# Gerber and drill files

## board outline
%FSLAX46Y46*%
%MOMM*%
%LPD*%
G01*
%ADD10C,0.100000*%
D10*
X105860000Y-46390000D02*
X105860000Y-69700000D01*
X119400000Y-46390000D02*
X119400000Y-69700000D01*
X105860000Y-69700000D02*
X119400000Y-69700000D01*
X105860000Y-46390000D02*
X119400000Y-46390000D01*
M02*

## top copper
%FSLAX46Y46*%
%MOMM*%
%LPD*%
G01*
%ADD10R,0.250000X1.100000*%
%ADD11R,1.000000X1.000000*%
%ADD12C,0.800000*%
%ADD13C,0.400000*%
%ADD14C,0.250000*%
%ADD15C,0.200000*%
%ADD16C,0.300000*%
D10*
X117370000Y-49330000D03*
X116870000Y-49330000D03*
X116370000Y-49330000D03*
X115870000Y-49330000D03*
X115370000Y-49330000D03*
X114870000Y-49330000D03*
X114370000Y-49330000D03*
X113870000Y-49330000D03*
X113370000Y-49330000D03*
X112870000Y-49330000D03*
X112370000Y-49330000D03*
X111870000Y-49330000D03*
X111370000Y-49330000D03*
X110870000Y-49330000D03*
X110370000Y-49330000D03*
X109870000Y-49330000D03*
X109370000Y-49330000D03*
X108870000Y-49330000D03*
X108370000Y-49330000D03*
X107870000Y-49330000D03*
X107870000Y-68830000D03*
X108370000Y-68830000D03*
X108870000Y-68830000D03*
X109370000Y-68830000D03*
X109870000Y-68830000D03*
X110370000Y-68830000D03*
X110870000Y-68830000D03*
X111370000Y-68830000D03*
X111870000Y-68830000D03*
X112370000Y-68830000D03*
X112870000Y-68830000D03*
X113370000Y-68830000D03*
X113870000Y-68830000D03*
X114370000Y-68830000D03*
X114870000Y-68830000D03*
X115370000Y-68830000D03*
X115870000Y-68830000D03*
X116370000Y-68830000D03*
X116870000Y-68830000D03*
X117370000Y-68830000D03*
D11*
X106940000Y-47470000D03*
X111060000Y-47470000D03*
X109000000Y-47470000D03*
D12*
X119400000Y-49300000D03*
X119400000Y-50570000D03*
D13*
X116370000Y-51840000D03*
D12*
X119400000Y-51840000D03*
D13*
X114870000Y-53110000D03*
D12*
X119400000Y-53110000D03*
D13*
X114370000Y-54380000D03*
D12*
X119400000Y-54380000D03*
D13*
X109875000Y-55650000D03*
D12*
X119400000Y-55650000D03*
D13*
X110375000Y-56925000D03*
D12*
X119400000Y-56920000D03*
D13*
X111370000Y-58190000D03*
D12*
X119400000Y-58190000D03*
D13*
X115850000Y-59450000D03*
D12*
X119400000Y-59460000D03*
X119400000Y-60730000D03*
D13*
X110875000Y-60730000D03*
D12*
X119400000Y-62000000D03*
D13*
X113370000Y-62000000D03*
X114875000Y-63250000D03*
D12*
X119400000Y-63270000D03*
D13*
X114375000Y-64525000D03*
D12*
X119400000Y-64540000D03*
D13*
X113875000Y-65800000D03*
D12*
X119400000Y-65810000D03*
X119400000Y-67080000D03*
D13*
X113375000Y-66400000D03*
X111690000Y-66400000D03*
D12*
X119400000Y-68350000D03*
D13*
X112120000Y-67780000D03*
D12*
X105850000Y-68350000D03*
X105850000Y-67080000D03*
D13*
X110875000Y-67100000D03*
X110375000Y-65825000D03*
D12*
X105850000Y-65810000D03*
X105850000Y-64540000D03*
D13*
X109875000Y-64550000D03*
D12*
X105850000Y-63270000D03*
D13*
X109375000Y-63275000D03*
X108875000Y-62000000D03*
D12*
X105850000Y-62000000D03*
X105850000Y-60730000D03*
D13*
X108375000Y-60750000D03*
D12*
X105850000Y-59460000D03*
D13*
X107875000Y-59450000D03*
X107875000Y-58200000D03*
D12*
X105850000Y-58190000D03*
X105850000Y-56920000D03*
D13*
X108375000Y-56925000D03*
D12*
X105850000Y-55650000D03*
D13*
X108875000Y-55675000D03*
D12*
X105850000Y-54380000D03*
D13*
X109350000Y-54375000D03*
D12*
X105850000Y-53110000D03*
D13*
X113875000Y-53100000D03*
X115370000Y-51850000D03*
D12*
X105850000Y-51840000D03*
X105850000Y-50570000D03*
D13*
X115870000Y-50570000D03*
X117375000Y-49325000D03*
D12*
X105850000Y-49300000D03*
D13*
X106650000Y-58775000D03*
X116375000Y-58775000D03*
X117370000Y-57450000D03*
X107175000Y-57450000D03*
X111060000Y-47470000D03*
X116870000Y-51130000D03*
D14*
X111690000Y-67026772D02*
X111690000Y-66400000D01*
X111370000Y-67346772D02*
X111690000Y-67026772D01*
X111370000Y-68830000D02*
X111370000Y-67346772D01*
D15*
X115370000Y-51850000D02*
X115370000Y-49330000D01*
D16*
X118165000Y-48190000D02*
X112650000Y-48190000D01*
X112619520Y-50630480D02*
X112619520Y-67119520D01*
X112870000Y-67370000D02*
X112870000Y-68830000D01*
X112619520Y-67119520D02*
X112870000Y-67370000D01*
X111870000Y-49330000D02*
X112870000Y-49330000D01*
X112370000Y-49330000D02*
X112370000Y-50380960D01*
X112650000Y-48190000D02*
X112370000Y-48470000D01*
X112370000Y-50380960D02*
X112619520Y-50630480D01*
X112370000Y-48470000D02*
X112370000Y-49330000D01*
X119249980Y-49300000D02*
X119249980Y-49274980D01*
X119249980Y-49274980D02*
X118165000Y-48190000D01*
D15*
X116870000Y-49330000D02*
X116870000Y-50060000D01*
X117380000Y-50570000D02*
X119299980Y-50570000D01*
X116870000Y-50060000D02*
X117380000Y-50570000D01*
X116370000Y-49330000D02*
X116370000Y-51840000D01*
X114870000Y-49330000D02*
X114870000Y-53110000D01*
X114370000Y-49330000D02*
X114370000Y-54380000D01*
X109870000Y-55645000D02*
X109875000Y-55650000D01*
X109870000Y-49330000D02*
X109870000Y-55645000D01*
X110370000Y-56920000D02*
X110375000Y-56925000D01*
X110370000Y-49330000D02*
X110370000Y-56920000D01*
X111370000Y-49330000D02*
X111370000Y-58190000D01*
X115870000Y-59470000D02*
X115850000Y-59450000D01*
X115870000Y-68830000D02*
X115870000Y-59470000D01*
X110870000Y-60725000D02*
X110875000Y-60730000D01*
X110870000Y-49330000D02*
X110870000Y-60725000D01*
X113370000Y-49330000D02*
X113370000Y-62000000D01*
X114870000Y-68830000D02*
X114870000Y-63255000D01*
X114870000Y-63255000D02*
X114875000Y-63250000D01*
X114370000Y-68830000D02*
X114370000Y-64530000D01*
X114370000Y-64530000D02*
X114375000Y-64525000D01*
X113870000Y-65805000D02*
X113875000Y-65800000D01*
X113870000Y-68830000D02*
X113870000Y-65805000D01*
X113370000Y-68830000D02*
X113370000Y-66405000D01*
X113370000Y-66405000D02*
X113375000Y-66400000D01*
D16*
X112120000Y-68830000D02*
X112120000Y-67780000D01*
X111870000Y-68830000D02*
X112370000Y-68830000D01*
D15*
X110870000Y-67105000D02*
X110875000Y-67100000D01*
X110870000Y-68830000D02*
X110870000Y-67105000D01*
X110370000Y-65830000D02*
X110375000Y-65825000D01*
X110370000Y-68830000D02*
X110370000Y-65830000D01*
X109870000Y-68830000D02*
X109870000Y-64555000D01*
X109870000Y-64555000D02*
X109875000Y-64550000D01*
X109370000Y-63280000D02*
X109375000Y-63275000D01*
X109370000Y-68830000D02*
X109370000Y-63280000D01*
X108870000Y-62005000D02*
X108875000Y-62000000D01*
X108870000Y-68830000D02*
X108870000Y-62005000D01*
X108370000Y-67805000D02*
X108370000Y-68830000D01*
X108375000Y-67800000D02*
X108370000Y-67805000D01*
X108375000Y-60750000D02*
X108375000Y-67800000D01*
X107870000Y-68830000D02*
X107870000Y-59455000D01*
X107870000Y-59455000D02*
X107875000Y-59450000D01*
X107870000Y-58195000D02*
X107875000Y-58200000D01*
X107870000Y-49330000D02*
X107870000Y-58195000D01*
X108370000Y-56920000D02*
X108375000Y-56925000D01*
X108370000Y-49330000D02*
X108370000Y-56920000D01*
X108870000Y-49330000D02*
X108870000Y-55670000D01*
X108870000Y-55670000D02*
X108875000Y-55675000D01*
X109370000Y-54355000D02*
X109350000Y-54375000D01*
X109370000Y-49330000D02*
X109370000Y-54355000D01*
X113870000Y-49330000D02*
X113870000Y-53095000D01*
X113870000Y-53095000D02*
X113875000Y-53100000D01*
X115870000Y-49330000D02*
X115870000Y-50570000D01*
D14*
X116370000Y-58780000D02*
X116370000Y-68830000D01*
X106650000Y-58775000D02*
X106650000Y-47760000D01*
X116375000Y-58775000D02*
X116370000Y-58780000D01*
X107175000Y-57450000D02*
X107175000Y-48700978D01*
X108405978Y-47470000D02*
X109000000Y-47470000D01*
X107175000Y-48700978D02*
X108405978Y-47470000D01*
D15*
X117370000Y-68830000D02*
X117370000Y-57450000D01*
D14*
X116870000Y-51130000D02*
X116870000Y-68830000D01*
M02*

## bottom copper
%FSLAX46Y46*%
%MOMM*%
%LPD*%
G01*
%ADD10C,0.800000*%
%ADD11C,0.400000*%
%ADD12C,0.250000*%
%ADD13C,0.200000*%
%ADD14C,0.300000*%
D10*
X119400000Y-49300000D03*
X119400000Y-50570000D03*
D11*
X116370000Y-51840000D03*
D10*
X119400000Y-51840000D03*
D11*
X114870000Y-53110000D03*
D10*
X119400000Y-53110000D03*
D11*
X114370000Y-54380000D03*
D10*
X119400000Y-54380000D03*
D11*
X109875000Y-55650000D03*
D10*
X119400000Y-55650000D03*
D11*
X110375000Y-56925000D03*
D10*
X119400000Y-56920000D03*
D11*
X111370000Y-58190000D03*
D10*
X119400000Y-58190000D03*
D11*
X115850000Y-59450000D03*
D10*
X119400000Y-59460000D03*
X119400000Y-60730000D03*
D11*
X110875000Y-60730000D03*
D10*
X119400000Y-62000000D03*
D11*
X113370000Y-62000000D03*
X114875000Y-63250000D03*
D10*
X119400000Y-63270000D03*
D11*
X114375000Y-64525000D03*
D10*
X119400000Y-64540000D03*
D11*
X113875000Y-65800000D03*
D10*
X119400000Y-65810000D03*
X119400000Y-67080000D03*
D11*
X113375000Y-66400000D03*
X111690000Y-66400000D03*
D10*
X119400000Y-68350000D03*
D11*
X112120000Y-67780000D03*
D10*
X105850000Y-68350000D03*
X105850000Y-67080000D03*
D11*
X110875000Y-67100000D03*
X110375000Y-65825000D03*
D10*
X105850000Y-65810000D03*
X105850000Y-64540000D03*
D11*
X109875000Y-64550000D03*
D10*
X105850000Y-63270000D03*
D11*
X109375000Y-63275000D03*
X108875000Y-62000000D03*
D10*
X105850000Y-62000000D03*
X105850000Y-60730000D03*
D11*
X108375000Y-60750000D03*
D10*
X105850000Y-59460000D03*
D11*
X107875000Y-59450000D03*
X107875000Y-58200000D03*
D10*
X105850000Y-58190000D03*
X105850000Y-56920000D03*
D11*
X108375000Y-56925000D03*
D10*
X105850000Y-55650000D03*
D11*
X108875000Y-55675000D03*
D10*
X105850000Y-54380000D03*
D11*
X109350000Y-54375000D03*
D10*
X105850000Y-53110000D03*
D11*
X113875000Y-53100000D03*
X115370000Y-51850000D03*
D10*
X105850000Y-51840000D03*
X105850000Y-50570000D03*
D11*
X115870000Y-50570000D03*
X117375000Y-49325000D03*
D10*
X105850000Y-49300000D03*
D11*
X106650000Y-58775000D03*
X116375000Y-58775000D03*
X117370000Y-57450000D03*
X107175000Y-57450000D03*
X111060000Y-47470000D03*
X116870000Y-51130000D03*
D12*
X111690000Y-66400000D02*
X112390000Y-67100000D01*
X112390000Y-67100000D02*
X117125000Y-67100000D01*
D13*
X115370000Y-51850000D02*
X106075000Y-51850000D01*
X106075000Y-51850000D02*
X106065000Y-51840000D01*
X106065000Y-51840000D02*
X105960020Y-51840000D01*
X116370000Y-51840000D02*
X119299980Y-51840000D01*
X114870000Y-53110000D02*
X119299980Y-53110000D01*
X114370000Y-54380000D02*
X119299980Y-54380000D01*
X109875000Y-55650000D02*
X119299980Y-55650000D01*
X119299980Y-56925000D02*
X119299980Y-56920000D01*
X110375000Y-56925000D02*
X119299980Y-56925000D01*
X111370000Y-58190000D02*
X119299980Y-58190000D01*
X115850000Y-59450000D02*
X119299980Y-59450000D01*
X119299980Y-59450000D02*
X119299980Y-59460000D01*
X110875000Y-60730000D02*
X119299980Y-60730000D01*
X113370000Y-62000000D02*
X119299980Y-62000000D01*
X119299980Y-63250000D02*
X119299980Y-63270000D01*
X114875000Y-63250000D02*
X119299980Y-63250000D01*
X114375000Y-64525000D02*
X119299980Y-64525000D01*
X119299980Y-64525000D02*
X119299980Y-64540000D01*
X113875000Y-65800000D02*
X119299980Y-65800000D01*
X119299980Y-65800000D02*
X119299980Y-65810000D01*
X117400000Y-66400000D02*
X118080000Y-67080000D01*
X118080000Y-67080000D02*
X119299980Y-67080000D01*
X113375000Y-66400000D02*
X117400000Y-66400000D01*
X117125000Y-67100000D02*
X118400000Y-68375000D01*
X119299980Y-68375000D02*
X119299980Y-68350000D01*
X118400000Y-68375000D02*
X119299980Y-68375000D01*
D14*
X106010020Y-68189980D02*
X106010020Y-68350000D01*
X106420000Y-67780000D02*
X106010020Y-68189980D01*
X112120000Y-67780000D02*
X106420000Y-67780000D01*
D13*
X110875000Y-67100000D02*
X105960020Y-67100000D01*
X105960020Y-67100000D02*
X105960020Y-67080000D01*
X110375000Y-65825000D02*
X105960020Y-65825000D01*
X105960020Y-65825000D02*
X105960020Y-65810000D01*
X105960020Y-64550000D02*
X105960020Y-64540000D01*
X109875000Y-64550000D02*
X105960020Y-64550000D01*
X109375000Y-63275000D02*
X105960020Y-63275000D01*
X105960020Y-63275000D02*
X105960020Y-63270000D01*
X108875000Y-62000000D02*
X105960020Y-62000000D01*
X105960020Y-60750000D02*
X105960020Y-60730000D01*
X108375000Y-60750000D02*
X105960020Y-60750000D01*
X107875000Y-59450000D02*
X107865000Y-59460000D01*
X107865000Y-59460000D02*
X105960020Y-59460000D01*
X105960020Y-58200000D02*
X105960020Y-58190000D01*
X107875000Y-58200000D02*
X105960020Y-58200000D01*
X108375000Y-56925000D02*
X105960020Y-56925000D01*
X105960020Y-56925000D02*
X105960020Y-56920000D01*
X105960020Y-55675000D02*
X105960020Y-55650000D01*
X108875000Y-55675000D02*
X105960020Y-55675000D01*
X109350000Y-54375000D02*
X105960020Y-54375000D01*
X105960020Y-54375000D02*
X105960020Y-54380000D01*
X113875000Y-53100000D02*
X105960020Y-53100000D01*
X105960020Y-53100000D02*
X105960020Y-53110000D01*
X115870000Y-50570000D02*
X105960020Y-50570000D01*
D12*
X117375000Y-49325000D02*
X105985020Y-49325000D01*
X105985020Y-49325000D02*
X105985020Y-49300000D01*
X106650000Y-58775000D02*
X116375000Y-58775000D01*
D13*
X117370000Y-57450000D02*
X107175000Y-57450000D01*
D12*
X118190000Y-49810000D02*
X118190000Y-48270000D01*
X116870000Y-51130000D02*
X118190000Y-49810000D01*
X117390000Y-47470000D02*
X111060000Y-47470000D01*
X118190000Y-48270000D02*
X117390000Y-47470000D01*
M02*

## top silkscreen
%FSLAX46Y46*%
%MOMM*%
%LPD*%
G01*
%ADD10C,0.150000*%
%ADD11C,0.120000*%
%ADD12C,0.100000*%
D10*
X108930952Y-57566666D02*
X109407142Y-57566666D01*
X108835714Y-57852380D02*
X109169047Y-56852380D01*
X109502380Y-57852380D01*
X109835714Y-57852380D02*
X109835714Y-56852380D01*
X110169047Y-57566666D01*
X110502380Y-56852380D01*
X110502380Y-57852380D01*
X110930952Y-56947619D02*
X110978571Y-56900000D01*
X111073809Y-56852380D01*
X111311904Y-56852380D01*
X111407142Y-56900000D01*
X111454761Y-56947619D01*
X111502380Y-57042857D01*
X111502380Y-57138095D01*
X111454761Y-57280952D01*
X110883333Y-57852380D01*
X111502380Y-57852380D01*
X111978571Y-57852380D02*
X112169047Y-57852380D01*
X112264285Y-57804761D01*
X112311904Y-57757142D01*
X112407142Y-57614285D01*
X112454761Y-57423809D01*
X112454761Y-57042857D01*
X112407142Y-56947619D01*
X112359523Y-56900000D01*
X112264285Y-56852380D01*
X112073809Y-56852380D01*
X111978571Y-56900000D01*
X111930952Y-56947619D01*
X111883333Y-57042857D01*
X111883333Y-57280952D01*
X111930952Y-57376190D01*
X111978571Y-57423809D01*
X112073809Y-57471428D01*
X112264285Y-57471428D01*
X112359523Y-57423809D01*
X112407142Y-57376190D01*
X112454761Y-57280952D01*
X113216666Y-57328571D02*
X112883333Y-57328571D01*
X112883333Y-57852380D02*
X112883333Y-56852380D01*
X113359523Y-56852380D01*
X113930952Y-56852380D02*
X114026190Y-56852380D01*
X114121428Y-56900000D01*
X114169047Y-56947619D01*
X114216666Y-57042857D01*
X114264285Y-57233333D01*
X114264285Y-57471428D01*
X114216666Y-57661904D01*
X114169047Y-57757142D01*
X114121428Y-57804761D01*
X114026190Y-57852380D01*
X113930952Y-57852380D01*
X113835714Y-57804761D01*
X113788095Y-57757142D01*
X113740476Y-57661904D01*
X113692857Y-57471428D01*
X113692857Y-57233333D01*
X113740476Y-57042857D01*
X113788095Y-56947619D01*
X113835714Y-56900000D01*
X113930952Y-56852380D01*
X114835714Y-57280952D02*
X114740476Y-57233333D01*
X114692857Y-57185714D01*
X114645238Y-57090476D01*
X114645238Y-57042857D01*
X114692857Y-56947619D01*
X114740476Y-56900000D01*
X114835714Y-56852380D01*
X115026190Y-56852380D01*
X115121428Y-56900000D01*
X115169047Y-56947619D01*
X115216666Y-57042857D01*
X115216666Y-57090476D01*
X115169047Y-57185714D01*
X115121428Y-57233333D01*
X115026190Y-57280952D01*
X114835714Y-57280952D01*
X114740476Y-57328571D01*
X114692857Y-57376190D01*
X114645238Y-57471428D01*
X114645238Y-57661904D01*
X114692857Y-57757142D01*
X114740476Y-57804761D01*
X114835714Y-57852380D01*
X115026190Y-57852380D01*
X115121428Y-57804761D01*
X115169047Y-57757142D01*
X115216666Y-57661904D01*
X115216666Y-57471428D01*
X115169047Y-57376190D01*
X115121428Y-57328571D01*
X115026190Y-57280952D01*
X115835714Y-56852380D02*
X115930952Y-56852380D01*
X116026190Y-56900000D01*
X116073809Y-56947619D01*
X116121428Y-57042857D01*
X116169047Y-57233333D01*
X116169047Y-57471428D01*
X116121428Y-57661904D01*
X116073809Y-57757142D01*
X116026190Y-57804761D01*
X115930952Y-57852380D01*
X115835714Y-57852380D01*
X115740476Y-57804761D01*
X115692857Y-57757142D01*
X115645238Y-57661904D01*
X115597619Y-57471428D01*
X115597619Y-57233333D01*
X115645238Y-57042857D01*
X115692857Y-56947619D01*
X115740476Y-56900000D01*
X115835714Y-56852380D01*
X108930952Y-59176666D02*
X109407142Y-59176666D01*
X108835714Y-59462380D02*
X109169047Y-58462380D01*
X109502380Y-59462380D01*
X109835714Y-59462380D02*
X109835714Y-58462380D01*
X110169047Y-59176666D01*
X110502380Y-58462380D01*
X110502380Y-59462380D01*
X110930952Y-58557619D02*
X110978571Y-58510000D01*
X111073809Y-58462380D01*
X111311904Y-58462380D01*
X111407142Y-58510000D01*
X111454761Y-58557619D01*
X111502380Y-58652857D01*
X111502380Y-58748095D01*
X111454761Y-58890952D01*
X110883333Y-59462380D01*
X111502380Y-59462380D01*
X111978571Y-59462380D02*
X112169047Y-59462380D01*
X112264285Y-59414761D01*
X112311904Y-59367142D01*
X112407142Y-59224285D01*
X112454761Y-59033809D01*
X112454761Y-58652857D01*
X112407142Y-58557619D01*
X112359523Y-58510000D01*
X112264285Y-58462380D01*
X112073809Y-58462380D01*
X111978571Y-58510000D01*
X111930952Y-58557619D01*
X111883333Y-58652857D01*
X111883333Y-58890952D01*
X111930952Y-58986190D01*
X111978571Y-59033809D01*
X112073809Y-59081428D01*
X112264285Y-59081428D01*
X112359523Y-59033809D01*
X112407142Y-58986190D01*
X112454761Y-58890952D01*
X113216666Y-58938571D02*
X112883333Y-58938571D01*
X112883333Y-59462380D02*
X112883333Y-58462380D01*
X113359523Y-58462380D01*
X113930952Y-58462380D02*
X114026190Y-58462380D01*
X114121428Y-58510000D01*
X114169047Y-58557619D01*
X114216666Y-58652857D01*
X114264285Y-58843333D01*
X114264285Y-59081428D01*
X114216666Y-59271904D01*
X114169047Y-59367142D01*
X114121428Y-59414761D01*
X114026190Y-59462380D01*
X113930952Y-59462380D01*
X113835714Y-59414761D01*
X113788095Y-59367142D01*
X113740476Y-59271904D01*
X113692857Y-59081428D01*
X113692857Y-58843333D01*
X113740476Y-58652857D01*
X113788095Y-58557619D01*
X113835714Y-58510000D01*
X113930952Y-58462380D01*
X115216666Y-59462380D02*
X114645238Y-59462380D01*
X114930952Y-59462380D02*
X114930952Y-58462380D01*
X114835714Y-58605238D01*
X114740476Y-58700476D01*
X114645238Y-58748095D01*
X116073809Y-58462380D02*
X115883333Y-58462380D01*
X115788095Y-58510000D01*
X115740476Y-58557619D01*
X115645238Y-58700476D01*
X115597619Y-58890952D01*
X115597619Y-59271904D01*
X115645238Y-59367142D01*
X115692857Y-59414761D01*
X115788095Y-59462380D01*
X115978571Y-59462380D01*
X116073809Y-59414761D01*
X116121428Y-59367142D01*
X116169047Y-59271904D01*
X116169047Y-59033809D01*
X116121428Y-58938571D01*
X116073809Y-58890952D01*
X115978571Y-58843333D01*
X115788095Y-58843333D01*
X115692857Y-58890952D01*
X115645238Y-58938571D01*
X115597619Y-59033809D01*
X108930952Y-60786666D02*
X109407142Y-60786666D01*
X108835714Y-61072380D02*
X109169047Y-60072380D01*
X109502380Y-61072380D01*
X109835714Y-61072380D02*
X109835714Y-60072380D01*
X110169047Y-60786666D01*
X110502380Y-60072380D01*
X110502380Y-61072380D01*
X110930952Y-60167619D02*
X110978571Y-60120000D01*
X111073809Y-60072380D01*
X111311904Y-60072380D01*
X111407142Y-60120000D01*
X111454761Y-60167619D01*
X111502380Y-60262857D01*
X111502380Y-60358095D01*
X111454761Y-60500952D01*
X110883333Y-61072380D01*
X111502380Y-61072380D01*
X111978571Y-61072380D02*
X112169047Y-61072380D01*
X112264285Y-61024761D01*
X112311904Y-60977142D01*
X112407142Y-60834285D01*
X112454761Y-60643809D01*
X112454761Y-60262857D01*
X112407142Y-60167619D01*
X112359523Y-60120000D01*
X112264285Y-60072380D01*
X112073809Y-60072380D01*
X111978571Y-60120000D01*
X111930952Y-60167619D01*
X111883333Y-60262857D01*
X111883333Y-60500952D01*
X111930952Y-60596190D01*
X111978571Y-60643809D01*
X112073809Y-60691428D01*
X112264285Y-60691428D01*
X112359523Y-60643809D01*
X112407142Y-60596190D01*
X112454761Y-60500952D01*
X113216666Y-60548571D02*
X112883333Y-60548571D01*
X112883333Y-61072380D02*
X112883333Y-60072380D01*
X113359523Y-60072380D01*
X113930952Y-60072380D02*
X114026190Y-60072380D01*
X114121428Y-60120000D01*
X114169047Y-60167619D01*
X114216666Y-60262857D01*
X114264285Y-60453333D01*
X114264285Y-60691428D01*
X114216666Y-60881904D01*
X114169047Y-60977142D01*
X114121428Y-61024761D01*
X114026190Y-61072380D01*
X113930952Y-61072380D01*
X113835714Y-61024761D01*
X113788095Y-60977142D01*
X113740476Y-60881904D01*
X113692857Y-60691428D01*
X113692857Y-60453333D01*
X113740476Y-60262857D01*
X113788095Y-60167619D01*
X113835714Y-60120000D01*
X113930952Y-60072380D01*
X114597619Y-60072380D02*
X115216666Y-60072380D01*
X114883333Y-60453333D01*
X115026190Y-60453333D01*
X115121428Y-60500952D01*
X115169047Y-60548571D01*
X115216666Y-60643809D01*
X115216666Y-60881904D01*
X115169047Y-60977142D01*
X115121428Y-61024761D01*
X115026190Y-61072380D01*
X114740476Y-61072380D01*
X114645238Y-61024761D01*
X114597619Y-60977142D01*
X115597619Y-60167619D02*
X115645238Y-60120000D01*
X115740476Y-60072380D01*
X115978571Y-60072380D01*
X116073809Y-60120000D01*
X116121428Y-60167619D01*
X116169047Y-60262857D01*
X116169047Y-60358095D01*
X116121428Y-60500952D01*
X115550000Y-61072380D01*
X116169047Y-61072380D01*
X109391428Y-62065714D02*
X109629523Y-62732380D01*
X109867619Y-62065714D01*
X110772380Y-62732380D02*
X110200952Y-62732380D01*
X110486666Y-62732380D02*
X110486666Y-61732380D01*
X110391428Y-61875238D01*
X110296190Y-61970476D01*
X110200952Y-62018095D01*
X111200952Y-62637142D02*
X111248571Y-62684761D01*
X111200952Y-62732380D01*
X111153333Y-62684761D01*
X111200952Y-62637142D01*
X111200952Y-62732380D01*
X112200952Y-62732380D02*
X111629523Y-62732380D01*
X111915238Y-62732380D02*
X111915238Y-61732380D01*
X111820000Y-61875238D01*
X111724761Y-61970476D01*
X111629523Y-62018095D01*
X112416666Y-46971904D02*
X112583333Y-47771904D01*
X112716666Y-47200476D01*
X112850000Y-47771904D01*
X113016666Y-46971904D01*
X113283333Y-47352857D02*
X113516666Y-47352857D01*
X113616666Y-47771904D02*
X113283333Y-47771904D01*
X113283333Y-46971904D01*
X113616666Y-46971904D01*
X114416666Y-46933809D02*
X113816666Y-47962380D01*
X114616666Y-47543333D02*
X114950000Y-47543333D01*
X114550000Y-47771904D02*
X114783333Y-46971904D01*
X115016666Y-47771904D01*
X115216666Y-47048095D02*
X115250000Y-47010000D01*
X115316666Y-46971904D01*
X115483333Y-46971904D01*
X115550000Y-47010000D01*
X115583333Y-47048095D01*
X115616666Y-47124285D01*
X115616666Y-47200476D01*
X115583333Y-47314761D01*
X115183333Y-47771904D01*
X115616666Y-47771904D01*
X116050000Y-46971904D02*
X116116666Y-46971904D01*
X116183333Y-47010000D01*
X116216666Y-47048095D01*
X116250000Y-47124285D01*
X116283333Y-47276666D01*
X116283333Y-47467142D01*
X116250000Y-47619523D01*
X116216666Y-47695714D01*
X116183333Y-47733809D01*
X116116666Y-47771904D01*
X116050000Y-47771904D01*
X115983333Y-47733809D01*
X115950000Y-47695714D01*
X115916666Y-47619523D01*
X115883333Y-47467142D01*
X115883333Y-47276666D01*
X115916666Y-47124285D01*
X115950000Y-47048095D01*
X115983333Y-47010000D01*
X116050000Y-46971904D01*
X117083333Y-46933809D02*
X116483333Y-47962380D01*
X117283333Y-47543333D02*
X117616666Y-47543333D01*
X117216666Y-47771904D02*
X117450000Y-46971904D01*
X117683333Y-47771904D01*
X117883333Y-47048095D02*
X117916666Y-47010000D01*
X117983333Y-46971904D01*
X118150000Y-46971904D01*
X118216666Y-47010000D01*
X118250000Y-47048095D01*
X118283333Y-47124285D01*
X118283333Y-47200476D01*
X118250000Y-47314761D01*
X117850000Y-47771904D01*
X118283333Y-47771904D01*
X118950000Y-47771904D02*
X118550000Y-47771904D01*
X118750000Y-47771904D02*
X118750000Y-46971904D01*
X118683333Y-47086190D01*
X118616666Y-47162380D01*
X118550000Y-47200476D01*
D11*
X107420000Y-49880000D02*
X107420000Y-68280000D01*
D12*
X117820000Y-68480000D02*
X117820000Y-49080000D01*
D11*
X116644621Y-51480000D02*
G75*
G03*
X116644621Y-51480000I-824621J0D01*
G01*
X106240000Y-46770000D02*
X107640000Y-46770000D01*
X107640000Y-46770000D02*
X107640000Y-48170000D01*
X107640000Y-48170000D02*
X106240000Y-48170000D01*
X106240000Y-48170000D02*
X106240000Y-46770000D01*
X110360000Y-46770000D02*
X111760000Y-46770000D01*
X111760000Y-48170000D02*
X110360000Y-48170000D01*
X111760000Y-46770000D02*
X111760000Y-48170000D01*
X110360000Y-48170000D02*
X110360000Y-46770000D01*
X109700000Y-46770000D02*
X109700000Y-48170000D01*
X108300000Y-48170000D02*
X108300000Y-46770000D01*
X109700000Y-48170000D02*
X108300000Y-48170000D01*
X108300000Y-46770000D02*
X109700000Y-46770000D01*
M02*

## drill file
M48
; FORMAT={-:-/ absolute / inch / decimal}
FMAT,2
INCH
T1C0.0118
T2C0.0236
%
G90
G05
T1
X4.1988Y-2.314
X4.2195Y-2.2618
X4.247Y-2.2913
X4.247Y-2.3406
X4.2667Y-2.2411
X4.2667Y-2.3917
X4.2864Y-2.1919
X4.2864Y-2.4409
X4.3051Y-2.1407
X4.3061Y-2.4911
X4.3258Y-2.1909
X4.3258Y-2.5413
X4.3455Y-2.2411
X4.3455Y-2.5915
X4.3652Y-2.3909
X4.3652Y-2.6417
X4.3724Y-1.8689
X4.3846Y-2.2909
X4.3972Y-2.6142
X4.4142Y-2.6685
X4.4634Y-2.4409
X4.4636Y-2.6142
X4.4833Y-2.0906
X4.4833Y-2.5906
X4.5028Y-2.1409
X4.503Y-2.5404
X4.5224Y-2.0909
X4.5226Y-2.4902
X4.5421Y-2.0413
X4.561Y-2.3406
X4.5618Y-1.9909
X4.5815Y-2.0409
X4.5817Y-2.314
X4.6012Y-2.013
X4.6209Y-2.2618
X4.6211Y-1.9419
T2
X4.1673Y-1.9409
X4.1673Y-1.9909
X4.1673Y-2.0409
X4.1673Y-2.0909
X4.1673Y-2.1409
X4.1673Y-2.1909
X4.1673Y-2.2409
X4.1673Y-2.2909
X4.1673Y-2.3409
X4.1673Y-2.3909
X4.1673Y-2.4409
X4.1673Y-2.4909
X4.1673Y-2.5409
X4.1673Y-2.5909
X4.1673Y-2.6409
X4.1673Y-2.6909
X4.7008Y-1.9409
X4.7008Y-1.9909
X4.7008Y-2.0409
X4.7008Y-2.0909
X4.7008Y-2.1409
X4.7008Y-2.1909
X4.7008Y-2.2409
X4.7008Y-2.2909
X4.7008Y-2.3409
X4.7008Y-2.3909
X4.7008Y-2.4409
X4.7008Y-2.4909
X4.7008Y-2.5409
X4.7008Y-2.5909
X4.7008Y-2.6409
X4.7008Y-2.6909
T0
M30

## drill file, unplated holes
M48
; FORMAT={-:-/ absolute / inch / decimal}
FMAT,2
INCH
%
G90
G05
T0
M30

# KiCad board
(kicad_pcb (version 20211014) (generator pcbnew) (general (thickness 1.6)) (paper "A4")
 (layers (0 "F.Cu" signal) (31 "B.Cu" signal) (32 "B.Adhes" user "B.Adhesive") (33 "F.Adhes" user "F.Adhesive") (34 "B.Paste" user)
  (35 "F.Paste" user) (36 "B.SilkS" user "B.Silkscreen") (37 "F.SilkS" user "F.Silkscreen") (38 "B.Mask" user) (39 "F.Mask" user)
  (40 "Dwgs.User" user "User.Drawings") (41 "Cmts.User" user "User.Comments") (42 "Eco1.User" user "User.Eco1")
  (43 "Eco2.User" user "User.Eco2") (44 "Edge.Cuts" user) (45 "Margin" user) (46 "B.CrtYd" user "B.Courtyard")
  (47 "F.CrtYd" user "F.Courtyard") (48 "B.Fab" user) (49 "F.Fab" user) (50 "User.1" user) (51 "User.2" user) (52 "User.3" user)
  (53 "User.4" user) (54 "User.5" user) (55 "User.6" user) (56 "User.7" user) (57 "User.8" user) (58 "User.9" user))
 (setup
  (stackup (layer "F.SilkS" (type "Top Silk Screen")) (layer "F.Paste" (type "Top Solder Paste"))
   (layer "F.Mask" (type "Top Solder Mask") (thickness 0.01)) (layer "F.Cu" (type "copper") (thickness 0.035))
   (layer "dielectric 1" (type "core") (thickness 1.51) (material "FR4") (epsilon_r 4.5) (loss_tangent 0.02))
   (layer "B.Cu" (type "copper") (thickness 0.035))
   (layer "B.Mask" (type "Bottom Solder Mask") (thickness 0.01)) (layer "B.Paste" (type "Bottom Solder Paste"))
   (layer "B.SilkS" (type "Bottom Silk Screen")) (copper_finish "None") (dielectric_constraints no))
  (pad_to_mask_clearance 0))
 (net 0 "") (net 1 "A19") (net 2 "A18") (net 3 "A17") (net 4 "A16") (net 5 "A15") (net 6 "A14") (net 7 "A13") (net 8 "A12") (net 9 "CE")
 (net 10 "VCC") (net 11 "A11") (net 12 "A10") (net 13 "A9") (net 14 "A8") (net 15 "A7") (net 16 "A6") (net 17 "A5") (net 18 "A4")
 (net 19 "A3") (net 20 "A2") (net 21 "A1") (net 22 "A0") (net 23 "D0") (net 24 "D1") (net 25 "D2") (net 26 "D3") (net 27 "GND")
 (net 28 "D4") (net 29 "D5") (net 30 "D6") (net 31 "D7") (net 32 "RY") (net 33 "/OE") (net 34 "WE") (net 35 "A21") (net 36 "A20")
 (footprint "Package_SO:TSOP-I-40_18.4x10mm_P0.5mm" (layer "F.Cu") (at 112.62 59.08 -90)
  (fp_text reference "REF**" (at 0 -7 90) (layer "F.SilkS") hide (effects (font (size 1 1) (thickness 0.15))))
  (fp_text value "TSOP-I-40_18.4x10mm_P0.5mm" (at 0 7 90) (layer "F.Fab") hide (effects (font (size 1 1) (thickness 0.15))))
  (fp_line (start -9.2 5.2) (end 9.2 5.2) (layer "F.SilkS") (width 0.12))
  (fp_line (start 9.4 -5.2) (end -10 -5.2) (layer "F.SilkS") (width 0.1))
  (fp_circle (center -7.6 -3.2) (end -6.8 -3) (layer "F.SilkS") (width 0.12) (fill none))
  (pad "1" smd rect (at -9.75 -4.75 270) (size 1.1 0.25) (layers "F.Cu" "F.Paste" "F.Mask") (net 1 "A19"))
  (pad "2" smd rect (at -9.75 -4.25 270) (size 1.1 0.25) (layers "F.Cu" "F.Paste" "F.Mask") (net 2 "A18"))
  (pad "3" smd rect (at -9.75 -3.75 270) (size 1.1 0.25) (layers "F.Cu" "F.Paste" "F.Mask") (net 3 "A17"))
  (pad "4" smd rect (at -9.75 -3.25 270) (size 1.1 0.25) (layers "F.Cu" "F.Paste" "F.Mask") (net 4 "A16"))
  (pad "5" smd rect (at -9.75 -2.75 270) (size 1.1 0.25) (layers "F.Cu" "F.Paste" "F.Mask") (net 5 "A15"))
  (pad "6" smd rect (at -9.75 -2.25 270) (size 1.1 0.25) (layers "F.Cu" "F.Paste" "F.Mask") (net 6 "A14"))
  (pad "7" smd rect (at -9.75 -1.75 270) (size 1.1 0.25) (layers "F.Cu" "F.Paste" "F.Mask") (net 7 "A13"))
  (pad "8" smd rect (at -9.75 -1.25 270) (size 1.1 0.25) (layers "F.Cu" "F.Paste" "F.Mask") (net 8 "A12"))
  (pad "9" smd rect (at -9.75 -0.75 270) (size 1.1 0.25) (layers "F.Cu" "F.Paste" "F.Mask") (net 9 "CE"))
  (pad "10" smd rect (at -9.75 -0.25 270) (size 1.1 0.25) (layers "F.Cu" "F.Paste" "F.Mask") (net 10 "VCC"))
  (pad "11" smd rect (at -9.75 0.25 270) (size 1.1 0.25) (layers "F.Cu" "F.Paste" "F.Mask") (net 10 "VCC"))
  (pad "12" smd rect (at -9.75 0.75 270) (size 1.1 0.25) (layers "F.Cu" "F.Paste" "F.Mask") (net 10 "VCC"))
  (pad "13" smd rect (at -9.75 1.25 270) (size 1.1 0.25) (layers "F.Cu" "F.Paste" "F.Mask") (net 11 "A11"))
  (pad "14" smd rect (at -9.75 1.75 270) (size 1.1 0.25) (layers "F.Cu" "F.Paste" "F.Mask") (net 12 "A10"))
  (pad "15" smd rect (at -9.75 2.25 270) (size 1.1 0.25) (layers "F.Cu" "F.Paste" "F.Mask") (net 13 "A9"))
  (pad "16" smd rect (at -9.75 2.75 270) (size 1.1 0.25) (layers "F.Cu" "F.Paste" "F.Mask") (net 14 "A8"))
  (pad "17" smd rect (at -9.75 3.25 270) (size 1.1 0.25) (layers "F.Cu" "F.Paste" "F.Mask") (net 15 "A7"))
  (pad "18" smd rect (at -9.75 3.75 270) (size 1.1 0.25) (layers "F.Cu" "F.Paste" "F.Mask") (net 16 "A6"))
  (pad "19" smd rect (at -9.75 4.25 270) (size 1.1 0.25) (layers "F.Cu" "F.Paste" "F.Mask") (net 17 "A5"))
  (pad "20" smd rect (at -9.75 4.75 270) (size 1.1 0.25) (layers "F.Cu" "F.Paste" "F.Mask") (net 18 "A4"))
  (pad "21" smd rect (at 9.75 4.75 270) (size 1.1 0.25) (layers "F.Cu" "F.Paste" "F.Mask") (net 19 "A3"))
  (pad "22" smd rect (at 9.75 4.25 270) (size 1.1 0.25) (layers "F.Cu" "F.Paste" "F.Mask") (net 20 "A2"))
  (pad "23" smd rect (at 9.75 3.75 270) (size 1.1 0.25) (layers "F.Cu" "F.Paste" "F.Mask") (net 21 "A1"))
  (pad "24" smd rect (at 9.75 3.25 270) (size 1.1 0.25) (layers "F.Cu" "F.Paste" "F.Mask") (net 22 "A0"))
  (pad "25" smd rect (at 9.75 2.75 270) (size 1.1 0.25) (layers "F.Cu" "F.Paste" "F.Mask") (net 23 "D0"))
  (pad "26" smd rect (at 9.75 2.25 270) (size 1.1 0.25) (layers "F.Cu" "F.Paste" "F.Mask") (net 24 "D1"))
  (pad "27" smd rect (at 9.75 1.75 270) (size 1.1 0.25) (layers "F.Cu" "F.Paste" "F.Mask") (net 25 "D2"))
  (pad "28" smd rect (at 9.75 1.25 270) (size 1.1 0.25) (layers "F.Cu" "F.Paste" "F.Mask") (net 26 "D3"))
  (pad "29" smd rect (at 9.75 0.75 270) (size 1.1 0.25) (layers "F.Cu" "F.Paste" "F.Mask") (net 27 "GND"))
  (pad "30" smd rect (at 9.75 0.25 270) (size 1.1 0.25) (layers "F.Cu" "F.Paste" "F.Mask") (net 27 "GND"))
  (pad "31" smd rect (at 9.75 -0.25 270) (size 1.1 0.25) (layers "F.Cu" "F.Paste" "F.Mask") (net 10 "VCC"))
  (pad "32" smd rect (at 9.75 -0.75 270) (size 1.1 0.25) (layers "F.Cu" "F.Paste" "F.Mask") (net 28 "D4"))
  (pad "33" smd rect (at 9.75 -1.25 270) (size 1.1 0.25) (layers "F.Cu" "F.Paste" "F.Mask") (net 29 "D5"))
  (pad "34" smd rect (at 9.75 -1.75 270) (size 1.1 0.25) (layers "F.Cu" "F.Paste" "F.Mask") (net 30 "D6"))
  (pad "35" smd rect (at 9.75 -2.25 270) (size 1.1 0.25) (layers "F.Cu" "F.Paste" "F.Mask") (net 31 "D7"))
  (pad "36" smd rect (at 9.75 -2.75 270) (size 1.1 0.25) (layers "F.Cu" "F.Paste" "F.Mask") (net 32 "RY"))
  (pad "37" smd rect (at 9.75 -3.25 270) (size 1.1 0.25) (layers "F.Cu" "F.Paste" "F.Mask") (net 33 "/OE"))
  (pad "38" smd rect (at 9.75 -3.75 270) (size 1.1 0.25) (layers "F.Cu" "F.Paste" "F.Mask") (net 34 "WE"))
  (pad "39" smd rect (at 9.75 -4.25 270) (size 1.1 0.25) (layers "F.Cu" "F.Paste" "F.Mask") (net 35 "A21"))
  (pad "40" smd rect (at 9.75 -4.75 270) (size 1.1 0.25) (layers "F.Cu" "F.Paste" "F.Mask") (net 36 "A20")))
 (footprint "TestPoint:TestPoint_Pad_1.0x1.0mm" (layer "F.Cu") (at 106.94 47.47)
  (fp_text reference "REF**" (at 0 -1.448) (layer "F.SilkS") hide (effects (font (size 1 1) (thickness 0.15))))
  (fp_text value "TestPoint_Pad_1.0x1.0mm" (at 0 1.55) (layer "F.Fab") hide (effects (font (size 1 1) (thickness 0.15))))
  (fp_line (start -0.7 -0.7) (end 0.7 -0.7) (layer "F.SilkS") (width 0.12))
  (fp_line (start 0.7 -0.7) (end 0.7 0.7) (layer "F.SilkS") (width 0.12))
  (fp_line (start 0.7 0.7) (end -0.7 0.7) (layer "F.SilkS") (width 0.12))
  (fp_line (start -0.7 0.7) (end -0.7 -0.7) (layer "F.SilkS") (width 0.12))
  (pad "" smd rect (at 0 0) (size 1 1) (layers "F.Cu" "F.Mask") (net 34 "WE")))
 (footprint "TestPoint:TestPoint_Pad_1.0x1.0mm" (layer "F.Cu") (at 111.06 47.47)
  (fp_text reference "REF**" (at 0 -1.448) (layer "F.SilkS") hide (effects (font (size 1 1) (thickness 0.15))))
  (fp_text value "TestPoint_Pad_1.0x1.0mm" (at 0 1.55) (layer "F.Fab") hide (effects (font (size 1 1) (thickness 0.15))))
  (fp_line (start -0.7 -0.7) (end 0.7 -0.7) (layer "F.SilkS") (width 0.12))
  (fp_line (start 0.7 0.7) (end -0.7 0.7) (layer "F.SilkS") (width 0.12))
  (fp_line (start 0.7 -0.7) (end 0.7 0.7) (layer "F.SilkS") (width 0.12))
  (fp_line (start -0.7 0.7) (end -0.7 -0.7) (layer "F.SilkS") (width 0.12))
  (pad "" smd rect (at 0 0) (size 1 1) (layers "F.Cu" "F.Mask") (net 35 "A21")))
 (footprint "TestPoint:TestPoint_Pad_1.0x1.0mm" (layer "F.Cu") (at 109 47.47)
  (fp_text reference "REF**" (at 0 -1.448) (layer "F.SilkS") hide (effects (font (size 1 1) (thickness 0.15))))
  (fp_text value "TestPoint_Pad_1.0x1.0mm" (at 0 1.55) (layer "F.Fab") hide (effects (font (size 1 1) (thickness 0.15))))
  (fp_line (start 0.7 -0.7) (end 0.7 0.7) (layer "F.SilkS") (width 0.12))
  (fp_line (start -0.7 0.7) (end -0.7 -0.7) (layer "F.SilkS") (width 0.12))
  (fp_line (start 0.7 0.7) (end -0.7 0.7) (layer "F.SilkS") (width 0.12))
  (fp_line (start -0.7 -0.7) (end 0.7 -0.7) (layer "F.SilkS") (width 0.12))
  (pad "" smd rect (at 0 0) (size 1 1) (layers "F.Cu" "F.Mask") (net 36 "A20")))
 (gr_line (start 105.86 46.39) (end 105.86 69.7) (layer "Edge.Cuts") (width 0.1))
 (gr_line (start 119.4 46.39) (end 119.4 69.7) (layer "Edge.Cuts") (width 0.1))
 (gr_line (start 105.86 69.7) (end 119.4 69.7) (layer "Edge.Cuts") (width 0.1))
 (gr_line (start 105.86 46.39) (end 119.4 46.39) (layer "Edge.Cuts") (width 0.1))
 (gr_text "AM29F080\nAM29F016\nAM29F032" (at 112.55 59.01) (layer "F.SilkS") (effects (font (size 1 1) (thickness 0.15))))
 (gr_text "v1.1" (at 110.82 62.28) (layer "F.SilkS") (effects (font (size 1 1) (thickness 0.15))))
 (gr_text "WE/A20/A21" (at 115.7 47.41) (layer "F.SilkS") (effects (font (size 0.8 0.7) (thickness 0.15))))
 (segment (start 118.165 48.19) (end 112.65 48.19) (width 0.3) (layer "F.Cu") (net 10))
 (segment (start 112.61952 50.63048) (end 112.61952 67.11952) (width 0.3) (layer "F.Cu") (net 10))
 (segment (start 112.87 67.37) (end 112.87 68.83) (width 0.3) (layer "F.Cu") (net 10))
 (segment (start 112.61952 67.11952) (end 112.87 67.37) (width 0.3) (layer "F.Cu") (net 10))
 (segment (start 111.87 49.33) (end 112.87 49.33) (width 0.3) (layer "F.Cu") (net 10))
 (segment (start 112.37 49.33) (end 112.37 50.38096) (width 0.3) (layer "F.Cu") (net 10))
 (segment (start 112.65 48.19) (end 112.37 48.47) (width 0.3) (layer "F.Cu") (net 10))
 (segment (start 112.37 50.38096) (end 112.61952 50.63048) (width 0.3) (layer "F.Cu") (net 10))
 (segment (start 112.37 48.47) (end 112.37 49.33) (width 0.3) (layer "F.Cu") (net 10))
 (segment (start 119.24998 49.3) (end 119.24998 49.27498) (width 0.3) (layer "F.Cu") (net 10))
 (segment (start 119.24998 49.27498) (end 118.165 48.19) (width 0.3) (layer "F.Cu") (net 10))
 (via (at 119.4 49.3) (size 0.8) (drill 0.6) (layers "F.Cu" "B.Cu") (free) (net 10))
 (segment (start 116.87 49.33) (end 116.87 50.06) (width 0.2) (layer "F.Cu") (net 2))
 (segment (start 117.38 50.57) (end 119.29998 50.57) (width 0.2) (layer "F.Cu") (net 2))
 (segment (start 116.87 50.06) (end 117.38 50.57) (width 0.2) (layer "F.Cu") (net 2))
 (via (at 119.4 50.57) (size 0.8) (drill 0.6) (layers "F.Cu" "B.Cu") (free) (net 2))
 (segment (start 116.37 49.33) (end 116.37 51.84) (width 0.2) (layer "F.Cu") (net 3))
 (via (at 116.37 51.84) (size 0.4) (drill 0.3) (layers "F.Cu" "B.Cu") (free) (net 3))
 (via (at 119.4 51.84) (size 0.8) (drill 0.6) (layers "F.Cu" "B.Cu") (free) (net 3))
 (segment (start 116.37 51.84) (end 119.29998 51.84) (width 0.2) (layer "B.Cu") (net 3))
 (segment (start 114.87 49.33) (end 114.87 53.11) (width 0.2) (layer "F.Cu") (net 6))
 (via (at 114.87 53.11) (size 0.4) (drill 0.3) (layers "F.Cu" "B.Cu") (free) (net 6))
 (via (at 119.4 53.11) (size 0.8) (drill 0.6) (layers "F.Cu" "B.Cu") (free) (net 6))
 (segment (start 114.87 53.11) (end 119.29998 53.11) (width 0.2) (layer "B.Cu") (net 6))
 (segment (start 114.37 49.33) (end 114.37 54.38) (width 0.2) (layer "F.Cu") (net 7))
 (via (at 114.37 54.38) (size 0.4) (drill 0.3) (layers "F.Cu" "B.Cu") (free) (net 7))
 (via (at 119.4 54.38) (size 0.8) (drill 0.6) (layers "F.Cu" "B.Cu") (free) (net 7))
 (segment (start 114.37 54.38) (end 119.29998 54.38) (width 0.2) (layer "B.Cu") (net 7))
 (segment (start 109.87 55.645) (end 109.875 55.65) (width 0.2) (layer "F.Cu") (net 14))
 (segment (start 109.87 49.33) (end 109.87 55.645) (width 0.2) (layer "F.Cu") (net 14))
 (via (at 109.875 55.65) (size 0.4) (drill 0.3) (layers "F.Cu" "B.Cu") (free) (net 14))
 (via (at 119.4 55.65) (size 0.8) (drill 0.6) (layers "F.Cu" "B.Cu") (free) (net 14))
 (segment (start 109.875 55.65) (end 119.29998 55.65) (width 0.2) (layer "B.Cu") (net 14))
 (segment (start 110.37 56.92) (end 110.375 56.925) (width 0.2) (layer "F.Cu") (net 13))
 (segment (start 110.37 49.33) (end 110.37 56.92) (width 0.2) (layer "F.Cu") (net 13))
 (via (at 110.375 56.925) (size 0.4) (drill 0.3) (layers "F.Cu" "B.Cu") (free) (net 13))
 (via (at 119.4 56.92) (size 0.8) (drill 0.6) (layers "F.Cu" "B.Cu") (free) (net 13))
 (segment (start 119.29998 56.925) (end 119.29998 56.92) (width 0.2) (layer "B.Cu") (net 13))
 (segment (start 110.375 56.925) (end 119.29998 56.925) (width 0.2) (layer "B.Cu") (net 13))
 (segment (start 111.37 49.33) (end 111.37 58.19) (width 0.2) (layer "F.Cu") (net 11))
 (via (at 111.37 58.19) (size 0.4) (drill 0.3) (layers "F.Cu" "B.Cu") (free) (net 11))
 (via (at 119.4 58.19) (size 0.8) (drill 0.6) (layers "F.Cu" "B.Cu") (free) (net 11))
 (segment (start 111.37 58.19) (end 119.29998 58.19) (width 0.2) (layer "B.Cu") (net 11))
 (segment (start 115.87 59.47) (end 115.85 59.45) (width 0.2) (layer "F.Cu") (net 33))
 (segment (start 115.87 68.83) (end 115.87 59.47) (width 0.2) (layer "F.Cu") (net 33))
 (via (at 115.85 59.45) (size 0.4) (drill 0.3) (layers "F.Cu" "B.Cu") (free) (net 33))
 (via (at 119.4 59.46) (size 0.8) (drill 0.6) (layers "F.Cu" "B.Cu") (free) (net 33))
 (segment (start 115.85 59.45) (end 119.29998 59.45) (width 0.2) (layer "B.Cu") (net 33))
 (segment (start 119.29998 59.45) (end 119.29998 59.46) (width 0.2) (layer "B.Cu") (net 33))
 (segment (start 110.87 60.725) (end 110.875 60.73) (width 0.2) (layer "F.Cu") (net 12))
 (segment (start 110.87 49.33) (end 110.87 60.725) (width 0.2) (layer "F.Cu") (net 12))
 (via (at 119.4 60.73) (size 0.8) (drill 0.6) (layers "F.Cu" "B.Cu") (free) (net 12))
 (via (at 110.875 60.73) (size 0.4) (drill 0.3) (layers "F.Cu" "B.Cu") (free) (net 12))
 (segment (start 110.875 60.73) (end 119.29998 60.73) (width 0.2) (layer "B.Cu") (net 12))
 (segment (start 113.37 49.33) (end 113.37 62) (width 0.2) (layer "F.Cu") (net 9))
 (via (at 119.4 62) (size 0.8) (drill 0.6) (layers "F.Cu" "B.Cu") (free) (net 9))
 (via (at 113.37 62) (size 0.4) (drill 0.3) (layers "F.Cu" "B.Cu") (free) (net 9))
 (segment (start 113.37 62) (end 119.29998 62) (width 0.2) (layer "B.Cu") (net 9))
 (segment (start 114.87 68.83) (end 114.87 63.255) (width 0.2) (layer "F.Cu") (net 31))
 (segment (start 114.87 63.255) (end 114.875 63.25) (width 0.2) (layer "F.Cu") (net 31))
 (via (at 114.875 63.25) (size 0.4) (drill 0.3) (layers "F.Cu" "B.Cu") (free) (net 31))
 (via (at 119.4 63.27) (size 0.8) (drill 0.6) (layers "F.Cu" "B.Cu") (free) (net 31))
 (segment (start 119.29998 63.25) (end 119.29998 63.27) (width 0.2) (layer "B.Cu") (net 31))
 (segment (start 114.875 63.25) (end 119.29998 63.25) (width 0.2) (layer "B.Cu") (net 31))
 (segment (start 114.37 68.83) (end 114.37 64.53) (width 0.2) (layer "F.Cu") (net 30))
 (segment (start 114.37 64.53) (end 114.375 64.525) (width 0.2) (layer "F.Cu") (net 30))
 (via (at 114.375 64.525) (size 0.4) (drill 0.3) (layers "F.Cu" "B.Cu") (free) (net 30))
 (via (at 119.4 64.54) (size 0.8) (drill 0.6) (layers "F.Cu" "B.Cu") (free) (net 30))
 (segment (start 114.375 64.525) (end 119.29998 64.525) (width 0.2) (layer "B.Cu") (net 30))
 (segment (start 119.29998 64.525) (end 119.29998 64.54) (width 0.2) (layer "B.Cu") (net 30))
 (segment (start 113.87 65.805) (end 113.875 65.8) (width 0.2) (layer "F.Cu") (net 29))
 (segment (start 113.87 68.83) (end 113.87 65.805) (width 0.2) (layer "F.Cu") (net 29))
 (via (at 113.875 65.8) (size 0.4) (drill 0.3) (layers "F.Cu" "B.Cu") (free) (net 29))
 (via (at 119.4 65.81) (size 0.8) (drill 0.6) (layers "F.Cu" "B.Cu") (free) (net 29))
 (segment (start 113.875 65.8) (end 119.29998 65.8) (width 0.2) (layer "B.Cu") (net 29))
 (segment (start 119.29998 65.8) (end 119.29998 65.81) (width 0.2) (layer "B.Cu") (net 29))
 (segment (start 113.37 68.83) (end 113.37 66.405) (width 0.2) (layer "F.Cu") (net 28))
 (segment (start 113.37 66.405) (end 113.375 66.4) (width 0.2) (layer "F.Cu") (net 28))
 (via (at 119.4 67.08) (size 0.8) (drill 0.6) (layers "F.Cu" "B.Cu") (free) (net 28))
 (via (at 113.375 66.4) (size 0.4) (drill 0.3) (layers "F.Cu" "B.Cu") (free) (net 28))
 (segment (start 117.4 66.4) (end 118.08 67.08) (width 0.2) (layer "B.Cu") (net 28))
 (segment (start 118.08 67.08) (end 119.29998 67.08) (width 0.2) (layer "B.Cu") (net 28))
 (segment (start 113.375 66.4) (end 117.4 66.4) (width 0.2) (layer "B.Cu") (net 28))
 (segment (start 111.37 67.346772) (end 111.69 67.026772) (width 0.25) (layer "F.Cu") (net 26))
 (segment (start 111.69 67.026772) (end 111.69 66.4) (width 0.25) (layer "F.Cu") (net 26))
 (segment (start 111.37 68.83) (end 111.37 67.346772) (width 0.25) (layer "F.Cu") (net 26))
 (via (at 111.69 66.4) (size 0.4) (drill 0.3) (layers "F.Cu" "B.Cu") (free) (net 26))
 (via (at 119.4 68.35) (size 0.8) (drill 0.6) (layers "F.Cu" "B.Cu") (free) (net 26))
 (segment (start 117.125 67.1) (end 118.4 68.375) (width 0.2) (layer "B.Cu") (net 26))
 (segment (start 119.29998 68.375) (end 119.29998 68.35) (width 0.2) (layer "B.Cu") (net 26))
 (segment (start 111.69 66.4) (end 112.39 67.1) (width 0.25) (layer "B.Cu") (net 26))
 (segment (start 118.4 68.375) (end 119.29998 68.375) (width 0.2) (layer "B.Cu") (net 26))
 (segment (start 112.39 67.1) (end 117.125 67.1) (width 0.25) (layer "B.Cu") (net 26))
 (segment (start 112.12 68.83) (end 112.12 67.78) (width 0.3) (layer "F.Cu") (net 27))
 (segment (start 111.87 68.83) (end 112.37 68.83) (width 0.3) (layer "F.Cu") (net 27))
 (via (at 112.12 67.78) (size 0.4) (drill 0.3) (layers "F.Cu" "B.Cu") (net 27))
 (via (at 105.85 68.35) (size 0.8) (drill 0.6) (layers "F.Cu" "B.Cu") (free) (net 27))
 (segment (start 106.01002 68.18998) (end 106.01002 68.35) (width 0.3) (layer "B.Cu") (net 27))
 (segment (start 106.42 67.78) (end 106.01002 68.18998) (width 0.3) (layer "B.Cu") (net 27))
 (segment (start 112.12 67.78) (end 106.42 67.78) (width 0.3) (layer "B.Cu") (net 27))
 (segment (start 110.87 67.105) (end 110.875 67.1) (width 0.2) (layer "F.Cu") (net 25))
 (segment (start 110.87 68.83) (end 110.87 67.105) (width 0.2) (layer "F.Cu") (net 25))
 (via (at 105.85 67.08) (size 0.8) (drill 0.6) (layers "F.Cu" "B.Cu") (free) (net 25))
 (via (at 110.875 67.1) (size 0.4) (drill 0.3) (layers "F.Cu" "B.Cu") (free) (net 25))
 (segment (start 110.875 67.1) (end 105.96002 67.1) (width 0.2) (layer "B.Cu") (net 25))
 (segment (start 105.96002 67.1) (end 105.96002 67.08) (width 0.2) (layer "B.Cu") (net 25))
 (segment (start 110.37 65.83) (end 110.375 65.825) (width 0.2) (layer "F.Cu") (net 24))
 (segment (start 110.37 68.83) (end 110.37 65.83) (width 0.2) (layer "F.Cu") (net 24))
 (via (at 110.375 65.825) (size 0.4) (drill 0.3) (layers "F.Cu" "B.Cu") (free) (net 24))
 (via (at 105.85 65.81) (size 0.8) (drill 0.6) (layers "F.Cu" "B.Cu") (free) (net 24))
 (segment (start 110.375 65.825) (end 105.96002 65.825) (width 0.2) (layer "B.Cu") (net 24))
 (segment (start 105.96002 65.825) (end 105.96002 65.81) (width 0.2) (layer "B.Cu") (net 24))
 (segment (start 109.87 68.83) (end 109.87 64.555) (width 0.2) (layer "F.Cu") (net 23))
 (segment (start 109.87 64.555) (end 109.875 64.55) (width 0.2) (layer "F.Cu") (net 23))
 (via (at 105.85 64.54) (size 0.8) (drill 0.6) (layers "F.Cu" "B.Cu") (free) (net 23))
 (via (at 109.875 64.55) (size 0.4) (drill 0.3) (layers "F.Cu" "B.Cu") (free) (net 23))
 (segment (start 105.96002 64.55) (end 105.96002 64.54) (width 0.2) (layer "B.Cu") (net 23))
 (segment (start 109.875 64.55) (end 105.96002 64.55) (width 0.2) (layer "B.Cu") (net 23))
 (segment (start 109.37 63.28) (end 109.375 63.275) (width 0.2) (layer "F.Cu") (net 22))
 (segment (start 109.37 68.83) (end 109.37 63.28) (width 0.2) (layer "F.Cu") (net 22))
 (via (at 105.85 63.27) (size 0.8) (drill 0.6) (layers "F.Cu" "B.Cu") (free) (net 22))
 (via (at 109.375 63.275) (size 0.4) (drill 0.3) (layers "F.Cu" "B.Cu") (free) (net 22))
 (segment (start 109.375 63.275) (end 105.96002 63.275) (width 0.2) (layer "B.Cu") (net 22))
 (segment (start 105.96002 63.275) (end 105.96002 63.27) (width 0.2) (layer "B.Cu") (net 22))
 (segment (start 108.87 62.005) (end 108.875 62) (width 0.2) (layer "F.Cu") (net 21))
 (segment (start 108.87 68.83) (end 108.87 62.005) (width 0.2) (layer "F.Cu") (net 21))
 (via (at 108.875 62) (size 0.4) (drill 0.3) (layers "F.Cu" "B.Cu") (free) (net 21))
 (via (at 105.85 62) (size 0.8) (drill 0.6) (layers "F.Cu" "B.Cu") (free) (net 21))
 (segment (start 108.875 62) (end 105.96002 62) (width 0.2) (layer "B.Cu") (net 21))
 (segment (start 108.37 67.805) (end 108.37 68.83) (width 0.2) (layer "F.Cu") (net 20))
 (segment (start 108.375 67.8) (end 108.37 67.805) (width 0.2) (layer "F.Cu") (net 20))
 (segment (start 108.375 60.75) (end 108.375 67.8) (width 0.2) (layer "F.Cu") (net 20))
 (via (at 105.85 60.73) (size 0.8) (drill 0.6) (layers "F.Cu" "B.Cu") (free) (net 20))
 (via (at 108.375 60.75) (size 0.4) (drill 0.3) (layers "F.Cu" "B.Cu") (free) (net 20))
 (segment (start 105.96002 60.75) (end 105.96002 60.73) (width 0.2) (layer "B.Cu") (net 20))
 (segment (start 108.375 60.75) (end 105.96002 60.75) (width 0.2) (layer "B.Cu") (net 20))
 (segment (start 107.87 68.83) (end 107.87 59.455) (width 0.2) (layer "F.Cu") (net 19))
 (segment (start 107.87 59.455) (end 107.875 59.45) (width 0.2) (layer "F.Cu") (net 19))
 (via (at 105.85 59.46) (size 0.8) (drill 0.6) (layers "F.Cu" "B.Cu") (free) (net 19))
 (via (at 107.875 59.45) (size 0.4) (drill 0.3) (layers "F.Cu" "B.Cu") (free) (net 19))
 (segment (start 107.875 59.45) (end 107.865 59.46) (width 0.2) (layer "B.Cu") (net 19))
 (segment (start 107.865 59.46) (end 105.96002 59.46) (width 0.2) (layer "B.Cu") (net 19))
 (segment (start 107.87 58.195) (end 107.875 58.2) (width 0.2) (layer "F.Cu") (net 18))
 (segment (start 107.87 49.33) (end 107.87 58.195) (width 0.2) (layer "F.Cu") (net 18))
 (via (at 107.875 58.2) (size 0.4) (drill 0.3) (layers "F.Cu" "B.Cu") (free) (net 18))
 (via (at 105.85 58.19) (size 0.8) (drill 0.6) (layers "F.Cu" "B.Cu") (free) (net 18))
 (segment (start 105.96002 58.2) (end 105.96002 58.19) (width 0.2) (layer "B.Cu") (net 18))
 (segment (start 107.875 58.2) (end 105.96002 58.2) (width 0.2) (layer "B.Cu") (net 18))
 (segment (start 108.37 56.92) (end 108.375 56.925) (width 0.2) (layer "F.Cu") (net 17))
 (segment (start 108.37 49.33) (end 108.37 56.92) (width 0.2) (layer "F.Cu") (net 17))
 (via (at 105.85 56.92) (size 0.8) (drill 0.6) (layers "F.Cu" "B.Cu") (free) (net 17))
 (via (at 108.375 56.925) (size 0.4) (drill 0.3) (layers "F.Cu" "B.Cu") (free) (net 17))
 (segment (start 108.375 56.925) (end 105.96002 56.925) (width 0.2) (layer "B.Cu") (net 17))
 (segment (start 105.96002 56.925) (end 105.96002 56.92) (width 0.2) (layer "B.Cu") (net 17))
 (segment (start 108.87 49.33) (end 108.87 55.67) (width 0.2) (layer "F.Cu") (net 16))
 (segment (start 108.87 55.67) (end 108.875 55.675) (width 0.2) (layer "F.Cu") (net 16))
 (via (at 105.85 55.65) (size 0.8) (drill 0.6) (layers "F.Cu" "B.Cu") (free) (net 16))
 (via (at 108.875 55.675) (size 0.4) (drill 0.3) (layers "F.Cu" "B.Cu") (free) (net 16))
 (segment (start 105.96002 55.675) (end 105.96002 55.65) (width 0.2) (layer "B.Cu") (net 16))
 (segment (start 108.875 55.675) (end 105.96002 55.675) (width 0.2) (layer "B.Cu") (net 16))
 (segment (start 109.37 54.355) (end 109.35 54.375) (width 0.2) (layer "F.Cu") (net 15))
 (segment (start 109.37 49.33) (end 109.37 54.355) (width 0.2) (layer "F.Cu") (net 15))
 (via (at 105.85 54.38) (size 0.8) (drill 0.6) (layers "F.Cu" "B.Cu") (free) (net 15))
 (via (at 109.35 54.375) (size 0.4) (drill 0.3) (layers "F.Cu" "B.Cu") (free) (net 15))
 (segment (start 109.35 54.375) (end 105.96002 54.375) (width 0.2) (layer "B.Cu") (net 15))
 (segment (start 105.96002 54.375) (end 105.96002 54.38) (width 0.2) (layer "B.Cu") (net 15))
 (segment (start 113.87 49.33) (end 113.87 53.095) (width 0.2) (layer "F.Cu") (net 8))
 (segment (start 113.87 53.095) (end 113.875 53.1) (width 0.2) (layer "F.Cu") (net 8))
 (via (at 105.85 53.11) (size 0.8) (drill 0.6) (layers "F.Cu" "B.Cu") (free) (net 8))
 (via (at 113.875 53.1) (size 0.4) (drill 0.3) (layers "F.Cu" "B.Cu") (free) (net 8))
 (segment (start 113.875 53.1) (end 105.96002 53.1) (width 0.2) (layer "B.Cu") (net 8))
 (segment (start 105.96002 53.1) (end 105.96002 53.11) (width 0.2) (layer "B.Cu") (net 8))
 (segment (start 115.37 51.85) (end 115.37 49.33) (width 0.2) (layer "F.Cu") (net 5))
 (via (at 115.37 51.85) (size 0.4) (drill 0.3) (layers "F.Cu" "B.Cu") (free) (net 5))
 (via (at 105.85 51.84) (size 0.8) (drill 0.6) (layers "F.Cu" "B.Cu") (free) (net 5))
 (segment (start 106.065 51.84) (end 105.96002 51.84) (width 0.2) (layer "B.Cu") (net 5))
 (segment (start 115.37 51.85) (end 106.075 51.85) (width 0.2) (layer "B.Cu") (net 5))
 (segment (start 106.075 51.85) (end 106.065 51.84) (width 0.2) (layer "B.Cu") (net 5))
 (segment (start 115.87 49.33) (end 115.87 50.57) (width 0.2) (layer "F.Cu") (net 4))
 (via (at 105.85 50.57) (size 0.8) (drill 0.6) (layers "F.Cu" "B.Cu") (free) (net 4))
 (via (at 115.87 50.57) (size 0.4) (drill 0.3) (layers "F.Cu" "B.Cu") (free) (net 4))
 (segment (start 115.87 50.57) (end 105.96002 50.57) (width 0.2) (layer "B.Cu") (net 4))
 (via (at 117.375 49.325) (size 0.4) (drill 0.3) (layers "F.Cu" "B.Cu") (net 1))
 (via (at 105.85 49.3) (size 0.8) (drill 0.6) (layers "F.Cu" "B.Cu") (free) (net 1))
 (segment (start 117.375 49.325) (end 105.98502 49.325) (width 0.25) (layer "B.Cu") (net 1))
 (segment (start 105.98502 49.325) (end 105.98502 49.3) (width 0.25) (layer "B.Cu") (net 1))
 (segment (start 116.37 58.78) (end 116.37 68.83) (width 0.25) (layer "F.Cu") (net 34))
 (segment (start 106.65 58.775) (end 106.65 47.76) (width 0.25) (layer "F.Cu") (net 34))
 (segment (start 116.375 58.775) (end 116.37 58.78) (width 0.25) (layer "F.Cu") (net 34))
 (via (at 106.65 58.775) (size 0.4) (drill 0.3) (layers "F.Cu" "B.Cu") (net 34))
 (via (at 116.375 58.775) (size 0.4) (drill 0.3) (layers "F.Cu" "B.Cu") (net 34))
 (segment (start 106.65 58.775) (end 116.375 58.775) (width 0.25) (layer "B.Cu") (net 34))
 (segment (start 107.175 57.45) (end 107.175 48.700978) (width 0.25) (layer "F.Cu") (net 36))
 (segment (start 108.405978 47.47) (end 109 47.47) (width 0.25) (layer "F.Cu") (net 36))
 (segment (start 107.175 48.700978) (end 108.405978 47.47) (width 0.25) (layer "F.Cu") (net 36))
 (segment (start 117.37 68.83) (end 117.37 57.45) (width 0.2) (layer "F.Cu") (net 36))
 (via (at 117.37 57.45) (size 0.4) (drill 0.3) (layers "F.Cu" "B.Cu") (free) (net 36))
 (via (at 107.175 57.45) (size 0.4) (drill 0.3) (layers "F.Cu" "B.Cu") (free) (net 36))
 (segment (start 117.37 57.45) (end 107.175 57.45) (width 0.2) (layer "B.Cu") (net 36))
 (segment (start 116.87 51.13) (end 116.87 68.83) (width 0.25) (layer "F.Cu") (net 35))
 (via (at 111.06 47.47) (size 0.4) (drill 0.3) (layers "F.Cu" "B.Cu") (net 35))
 (via (at 116.87 51.13) (size 0.4) (drill 0.3) (layers "F.Cu" "B.Cu") (free) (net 35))
 (segment (start 118.19 49.81) (end 118.19 48.27) (width 0.25) (layer "B.Cu") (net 35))
 (segment (start 116.87 51.13) (end 118.19 49.81) (width 0.25) (layer "B.Cu") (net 35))
 (segment (start 117.39 47.47) (end 111.06 47.47) (width 0.25) (layer "B.Cu") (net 35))
 (segment (start 118.19 48.27) (end 117.39 47.47) (width 0.25) (layer "B.Cu") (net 35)))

